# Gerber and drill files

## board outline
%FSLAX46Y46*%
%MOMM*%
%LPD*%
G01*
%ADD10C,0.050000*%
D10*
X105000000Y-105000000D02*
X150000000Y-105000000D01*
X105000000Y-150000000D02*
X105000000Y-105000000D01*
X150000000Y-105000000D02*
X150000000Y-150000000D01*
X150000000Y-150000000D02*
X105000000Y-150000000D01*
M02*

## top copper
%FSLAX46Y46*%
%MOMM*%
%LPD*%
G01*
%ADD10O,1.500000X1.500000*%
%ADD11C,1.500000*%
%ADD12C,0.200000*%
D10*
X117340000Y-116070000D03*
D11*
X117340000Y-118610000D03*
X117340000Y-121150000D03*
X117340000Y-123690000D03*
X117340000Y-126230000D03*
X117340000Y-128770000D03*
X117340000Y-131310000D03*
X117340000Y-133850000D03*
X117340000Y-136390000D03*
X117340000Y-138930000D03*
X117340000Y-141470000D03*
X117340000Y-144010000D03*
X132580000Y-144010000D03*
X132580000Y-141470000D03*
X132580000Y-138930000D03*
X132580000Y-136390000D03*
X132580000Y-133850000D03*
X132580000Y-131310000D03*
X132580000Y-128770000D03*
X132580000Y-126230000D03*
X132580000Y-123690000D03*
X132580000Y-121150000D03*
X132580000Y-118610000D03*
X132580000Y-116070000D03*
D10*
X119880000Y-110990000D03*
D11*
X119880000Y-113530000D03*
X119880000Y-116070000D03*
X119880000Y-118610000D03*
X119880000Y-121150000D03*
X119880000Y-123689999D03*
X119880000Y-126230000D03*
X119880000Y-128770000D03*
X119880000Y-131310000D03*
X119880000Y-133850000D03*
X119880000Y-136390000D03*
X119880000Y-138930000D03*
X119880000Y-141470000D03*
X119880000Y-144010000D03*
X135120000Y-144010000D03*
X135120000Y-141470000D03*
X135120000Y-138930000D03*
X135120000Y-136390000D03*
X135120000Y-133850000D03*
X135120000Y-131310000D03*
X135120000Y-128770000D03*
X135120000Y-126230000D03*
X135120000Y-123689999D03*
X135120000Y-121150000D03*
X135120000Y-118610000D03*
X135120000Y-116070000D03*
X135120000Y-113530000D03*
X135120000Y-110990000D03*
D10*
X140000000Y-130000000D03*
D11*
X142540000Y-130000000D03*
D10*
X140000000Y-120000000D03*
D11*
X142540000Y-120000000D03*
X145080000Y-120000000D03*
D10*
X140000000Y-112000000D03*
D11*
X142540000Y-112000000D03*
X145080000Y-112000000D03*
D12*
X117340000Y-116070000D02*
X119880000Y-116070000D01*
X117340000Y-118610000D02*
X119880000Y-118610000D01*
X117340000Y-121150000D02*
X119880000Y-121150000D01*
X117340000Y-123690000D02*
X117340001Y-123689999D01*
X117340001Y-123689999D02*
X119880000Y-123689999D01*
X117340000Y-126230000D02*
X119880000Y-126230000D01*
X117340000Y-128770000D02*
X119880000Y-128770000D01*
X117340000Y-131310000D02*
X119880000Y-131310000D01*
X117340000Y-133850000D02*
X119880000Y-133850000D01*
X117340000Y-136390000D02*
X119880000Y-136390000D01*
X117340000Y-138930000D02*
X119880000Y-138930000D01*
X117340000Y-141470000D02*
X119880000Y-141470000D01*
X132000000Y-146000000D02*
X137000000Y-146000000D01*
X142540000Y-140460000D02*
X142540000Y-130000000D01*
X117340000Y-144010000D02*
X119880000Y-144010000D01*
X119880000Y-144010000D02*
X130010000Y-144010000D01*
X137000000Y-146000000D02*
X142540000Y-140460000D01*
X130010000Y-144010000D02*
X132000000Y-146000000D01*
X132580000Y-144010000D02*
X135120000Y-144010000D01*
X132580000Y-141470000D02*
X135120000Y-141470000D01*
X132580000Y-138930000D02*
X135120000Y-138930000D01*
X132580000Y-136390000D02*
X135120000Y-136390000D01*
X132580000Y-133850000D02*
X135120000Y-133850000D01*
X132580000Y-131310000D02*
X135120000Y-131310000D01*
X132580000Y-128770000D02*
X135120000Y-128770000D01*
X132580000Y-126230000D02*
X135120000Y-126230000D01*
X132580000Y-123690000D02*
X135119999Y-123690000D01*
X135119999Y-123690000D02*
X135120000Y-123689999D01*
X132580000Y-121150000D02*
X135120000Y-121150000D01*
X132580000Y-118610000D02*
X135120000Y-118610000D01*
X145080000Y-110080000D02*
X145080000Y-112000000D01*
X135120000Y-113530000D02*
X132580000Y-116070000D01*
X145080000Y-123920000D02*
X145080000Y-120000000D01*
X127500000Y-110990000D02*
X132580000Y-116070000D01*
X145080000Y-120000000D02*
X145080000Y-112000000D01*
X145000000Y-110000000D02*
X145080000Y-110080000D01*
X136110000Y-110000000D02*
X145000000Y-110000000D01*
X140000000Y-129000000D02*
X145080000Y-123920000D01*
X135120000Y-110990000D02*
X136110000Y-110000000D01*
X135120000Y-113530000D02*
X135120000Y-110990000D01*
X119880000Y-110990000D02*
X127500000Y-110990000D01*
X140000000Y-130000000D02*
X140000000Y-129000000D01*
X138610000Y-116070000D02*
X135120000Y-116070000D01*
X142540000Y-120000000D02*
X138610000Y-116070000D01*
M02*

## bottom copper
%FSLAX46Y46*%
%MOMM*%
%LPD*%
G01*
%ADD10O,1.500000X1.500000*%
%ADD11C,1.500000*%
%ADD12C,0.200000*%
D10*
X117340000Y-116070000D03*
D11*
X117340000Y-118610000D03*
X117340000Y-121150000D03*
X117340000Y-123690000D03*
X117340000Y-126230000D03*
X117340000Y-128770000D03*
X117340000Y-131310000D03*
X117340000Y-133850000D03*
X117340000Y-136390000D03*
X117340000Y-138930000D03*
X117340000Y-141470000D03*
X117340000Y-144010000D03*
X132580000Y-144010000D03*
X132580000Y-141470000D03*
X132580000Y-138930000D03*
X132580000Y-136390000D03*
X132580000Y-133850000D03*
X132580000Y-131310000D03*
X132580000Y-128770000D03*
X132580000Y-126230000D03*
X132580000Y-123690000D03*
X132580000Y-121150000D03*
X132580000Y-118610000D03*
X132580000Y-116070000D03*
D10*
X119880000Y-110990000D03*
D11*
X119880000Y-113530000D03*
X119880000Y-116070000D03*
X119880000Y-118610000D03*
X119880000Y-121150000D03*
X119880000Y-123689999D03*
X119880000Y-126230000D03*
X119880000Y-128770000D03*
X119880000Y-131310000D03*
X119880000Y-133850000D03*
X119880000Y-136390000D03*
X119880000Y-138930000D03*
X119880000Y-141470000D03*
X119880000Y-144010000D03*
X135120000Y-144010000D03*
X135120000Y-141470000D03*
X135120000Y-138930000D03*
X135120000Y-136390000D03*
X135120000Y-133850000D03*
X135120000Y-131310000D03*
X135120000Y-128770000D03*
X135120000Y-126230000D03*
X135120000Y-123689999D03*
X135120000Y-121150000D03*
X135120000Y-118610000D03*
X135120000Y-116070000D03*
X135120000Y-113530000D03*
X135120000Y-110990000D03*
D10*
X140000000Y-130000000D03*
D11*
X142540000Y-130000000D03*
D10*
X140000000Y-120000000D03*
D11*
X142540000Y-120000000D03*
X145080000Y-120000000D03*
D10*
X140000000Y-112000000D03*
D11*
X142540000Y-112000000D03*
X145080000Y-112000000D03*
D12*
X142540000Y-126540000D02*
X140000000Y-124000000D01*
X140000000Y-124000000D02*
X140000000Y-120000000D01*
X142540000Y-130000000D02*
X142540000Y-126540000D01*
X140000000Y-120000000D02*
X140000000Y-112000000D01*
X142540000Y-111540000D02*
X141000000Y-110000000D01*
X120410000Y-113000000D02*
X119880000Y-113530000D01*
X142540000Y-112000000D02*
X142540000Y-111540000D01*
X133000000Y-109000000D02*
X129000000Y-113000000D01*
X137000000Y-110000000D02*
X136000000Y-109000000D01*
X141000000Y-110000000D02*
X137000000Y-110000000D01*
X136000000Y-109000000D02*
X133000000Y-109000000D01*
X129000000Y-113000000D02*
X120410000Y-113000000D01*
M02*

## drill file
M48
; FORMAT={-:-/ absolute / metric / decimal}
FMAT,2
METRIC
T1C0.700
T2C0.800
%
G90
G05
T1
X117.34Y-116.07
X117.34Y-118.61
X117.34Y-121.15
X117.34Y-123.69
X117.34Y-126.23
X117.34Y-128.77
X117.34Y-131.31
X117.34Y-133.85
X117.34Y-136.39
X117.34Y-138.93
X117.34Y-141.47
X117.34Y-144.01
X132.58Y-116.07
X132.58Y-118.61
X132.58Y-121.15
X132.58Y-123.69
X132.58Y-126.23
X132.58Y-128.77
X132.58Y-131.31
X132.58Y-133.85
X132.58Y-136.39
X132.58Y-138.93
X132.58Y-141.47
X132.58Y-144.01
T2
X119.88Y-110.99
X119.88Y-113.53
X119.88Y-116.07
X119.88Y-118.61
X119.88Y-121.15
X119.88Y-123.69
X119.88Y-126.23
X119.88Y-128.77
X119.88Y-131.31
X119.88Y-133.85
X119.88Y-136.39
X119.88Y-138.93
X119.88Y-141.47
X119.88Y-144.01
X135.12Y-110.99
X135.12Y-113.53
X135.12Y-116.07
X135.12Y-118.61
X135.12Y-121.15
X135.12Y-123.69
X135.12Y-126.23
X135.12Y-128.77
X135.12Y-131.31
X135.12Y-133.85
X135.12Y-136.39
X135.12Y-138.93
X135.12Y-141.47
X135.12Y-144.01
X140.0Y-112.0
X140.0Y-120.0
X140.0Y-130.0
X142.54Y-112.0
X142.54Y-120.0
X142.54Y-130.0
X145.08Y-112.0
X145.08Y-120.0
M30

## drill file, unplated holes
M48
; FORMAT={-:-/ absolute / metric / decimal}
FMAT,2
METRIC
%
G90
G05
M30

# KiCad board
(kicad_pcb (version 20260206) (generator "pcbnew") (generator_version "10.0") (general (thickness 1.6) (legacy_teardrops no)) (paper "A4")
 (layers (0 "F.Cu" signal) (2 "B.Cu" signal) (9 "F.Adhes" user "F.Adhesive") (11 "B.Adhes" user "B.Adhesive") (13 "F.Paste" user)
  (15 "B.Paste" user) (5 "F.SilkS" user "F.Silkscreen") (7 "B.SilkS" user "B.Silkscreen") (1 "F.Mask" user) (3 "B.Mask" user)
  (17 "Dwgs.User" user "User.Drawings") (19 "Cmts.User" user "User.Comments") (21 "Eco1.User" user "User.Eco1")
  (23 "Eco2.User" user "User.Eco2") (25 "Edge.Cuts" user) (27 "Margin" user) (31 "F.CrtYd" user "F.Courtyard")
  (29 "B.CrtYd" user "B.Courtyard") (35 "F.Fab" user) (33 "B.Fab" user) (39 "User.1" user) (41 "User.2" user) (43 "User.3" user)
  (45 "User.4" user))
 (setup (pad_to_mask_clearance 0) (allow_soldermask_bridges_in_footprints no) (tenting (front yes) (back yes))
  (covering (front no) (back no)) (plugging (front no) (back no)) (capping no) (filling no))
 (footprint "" (layer "F.Cu") (at 100 100)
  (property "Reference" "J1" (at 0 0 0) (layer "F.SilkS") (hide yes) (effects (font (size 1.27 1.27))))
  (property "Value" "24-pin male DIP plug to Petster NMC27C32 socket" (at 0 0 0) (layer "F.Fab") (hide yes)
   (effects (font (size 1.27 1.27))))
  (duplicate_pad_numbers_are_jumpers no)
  (pad "1" thru_hole oval (at 17.34 16.07) (size 1.5 1.5) (drill 0.7) (layers "*.Cu" "*.Mask") (remove_unused_layers no) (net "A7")
   (thermal_bridge_angle 45))
  (pad "2" thru_hole circle (at 17.34 18.61) (size 1.5 1.5) (drill 0.7) (layers "*.Cu" "*.Mask") (remove_unused_layers no) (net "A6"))
  (pad "3" thru_hole circle (at 17.34 21.15) (size 1.5 1.5) (drill 0.7) (layers "*.Cu" "*.Mask") (remove_unused_layers no) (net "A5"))
  (pad "4" thru_hole circle (at 17.34 23.69) (size 1.5 1.5) (drill 0.7) (layers "*.Cu" "*.Mask") (remove_unused_layers no) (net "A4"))
  (pad "5" thru_hole circle (at 17.34 26.23) (size 1.5 1.5) (drill 0.7) (layers "*.Cu" "*.Mask") (remove_unused_layers no) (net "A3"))
  (pad "6" thru_hole circle (at 17.34 28.77) (size 1.5 1.5) (drill 0.7) (layers "*.Cu" "*.Mask") (remove_unused_layers no) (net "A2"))
  (pad "7" thru_hole circle (at 17.34 31.31) (size 1.5 1.5) (drill 0.7) (layers "*.Cu" "*.Mask") (remove_unused_layers no) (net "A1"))
  (pad "8" thru_hole circle (at 17.34 33.85) (size 1.5 1.5) (drill 0.7) (layers "*.Cu" "*.Mask") (remove_unused_layers no) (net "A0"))
  (pad "9" thru_hole circle (at 17.34 36.39) (size 1.5 1.5) (drill 0.7) (layers "*.Cu" "*.Mask") (remove_unused_layers no) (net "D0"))
  (pad "10" thru_hole circle (at 17.34 38.93) (size 1.5 1.5) (drill 0.7) (layers "*.Cu" "*.Mask") (remove_unused_layers no) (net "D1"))
  (pad "11" thru_hole circle (at 17.34 41.47) (size 1.5 1.5) (drill 0.7) (layers "*.Cu" "*.Mask") (remove_unused_layers no) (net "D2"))
  (pad "12" thru_hole circle (at 17.34 44.01) (size 1.5 1.5) (drill 0.7) (layers "*.Cu" "*.Mask") (remove_unused_layers no) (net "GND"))
  (pad "13" thru_hole circle (at 32.58 44.01) (size 1.5 1.5) (drill 0.7) (layers "*.Cu" "*.Mask") (remove_unused_layers no) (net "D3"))
  (pad "14" thru_hole circle (at 32.58 41.47) (size 1.5 1.5) (drill 0.7) (layers "*.Cu" "*.Mask") (remove_unused_layers no) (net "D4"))
  (pad "15" thru_hole circle (at 32.58 38.93) (size 1.5 1.5) (drill 0.7) (layers "*.Cu" "*.Mask") (remove_unused_layers no) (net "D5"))
  (pad "16" thru_hole circle (at 32.58 36.39) (size 1.5 1.5) (drill 0.7) (layers "*.Cu" "*.Mask") (remove_unused_layers no) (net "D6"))
  (pad "17" thru_hole circle (at 32.58 33.85) (size 1.5 1.5) (drill 0.7) (layers "*.Cu" "*.Mask") (remove_unused_layers no) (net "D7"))
  (pad "18" thru_hole circle (at 32.58 31.31) (size 1.5 1.5) (drill 0.7) (layers "*.Cu" "*.Mask") (remove_unused_layers no) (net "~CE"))
  (pad "19" thru_hole circle (at 32.58 28.77) (size 1.5 1.5) (drill 0.7) (layers "*.Cu" "*.Mask") (remove_unused_layers no) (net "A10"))
  (pad "20" thru_hole circle (at 32.58 26.23) (size 1.5 1.5) (drill 0.7) (layers "*.Cu" "*.Mask") (remove_unused_layers no) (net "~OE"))
  (pad "21" thru_hole circle (at 32.58 23.69) (size 1.5 1.5) (drill 0.7) (layers "*.Cu" "*.Mask") (remove_unused_layers no) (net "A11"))
  (pad "22" thru_hole circle (at 32.58 21.15) (size 1.5 1.5) (drill 0.7) (layers "*.Cu" "*.Mask") (remove_unused_layers no) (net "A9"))
  (pad "23" thru_hole circle (at 32.58 18.61) (size 1.5 1.5) (drill 0.7) (layers "*.Cu" "*.Mask") (remove_unused_layers no) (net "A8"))
  (pad "24" thru_hole circle (at 32.58 16.07) (size 1.5 1.5) (drill 0.7) (layers "*.Cu" "*.Mask") (remove_unused_layers no) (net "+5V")))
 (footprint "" (layer "F.Cu") (at 100 100)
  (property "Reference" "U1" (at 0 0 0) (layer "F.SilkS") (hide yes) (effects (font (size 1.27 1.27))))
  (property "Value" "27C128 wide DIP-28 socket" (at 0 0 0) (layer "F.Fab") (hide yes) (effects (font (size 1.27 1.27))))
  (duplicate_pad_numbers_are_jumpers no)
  (pad "1" thru_hole oval (at 19.88 10.99) (size 1.5 1.5) (drill 0.8) (layers "*.Cu" "*.Mask") (remove_unused_layers no) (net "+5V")
   (thermal_bridge_angle 45))
  (pad "2" thru_hole circle (at 19.88 13.53) (size 1.5 1.5) (drill 0.8) (layers "*.Cu" "*.Mask") (remove_unused_layers no) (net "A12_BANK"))
  (pad "3" thru_hole circle (at 19.88 16.07) (size 1.5 1.5) (drill 0.8) (layers "*.Cu" "*.Mask") (remove_unused_layers no) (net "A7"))
  (pad "4" thru_hole circle (at 19.88 18.61) (size 1.5 1.5) (drill 0.8) (layers "*.Cu" "*.Mask") (remove_unused_layers no) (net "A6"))
  (pad "5" thru_hole circle (at 19.88 21.15) (size 1.5 1.5) (drill 0.8) (layers "*.Cu" "*.Mask") (remove_unused_layers no) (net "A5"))
  (pad "6" thru_hole circle (at 19.88 23.689999) (size 1.5 1.5) (drill 0.8) (layers "*.Cu" "*.Mask") (remove_unused_layers no) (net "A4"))
  (pad "7" thru_hole circle (at 19.88 26.23) (size 1.5 1.5) (drill 0.8) (layers "*.Cu" "*.Mask") (remove_unused_layers no) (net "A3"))
  (pad "8" thru_hole circle (at 19.88 28.77) (size 1.5 1.5) (drill 0.8) (layers "*.Cu" "*.Mask") (remove_unused_layers no) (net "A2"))
  (pad "9" thru_hole circle (at 19.88 31.31) (size 1.5 1.5) (drill 0.8) (layers "*.Cu" "*.Mask") (remove_unused_layers no) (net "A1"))
  (pad "10" thru_hole circle (at 19.88 33.85) (size 1.5 1.5) (drill 0.8) (layers "*.Cu" "*.Mask") (remove_unused_layers no) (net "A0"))
  (pad "11" thru_hole circle (at 19.88 36.39) (size 1.5 1.5) (drill 0.8) (layers "*.Cu" "*.Mask") (remove_unused_layers no) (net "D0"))
  (pad "12" thru_hole circle (at 19.88 38.93) (size 1.5 1.5) (drill 0.8) (layers "*.Cu" "*.Mask") (remove_unused_layers no) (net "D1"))
  (pad "13" thru_hole circle (at 19.88 41.47) (size 1.5 1.5) (drill 0.8) (layers "*.Cu" "*.Mask") (remove_unused_layers no) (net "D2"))
  (pad "14" thru_hole circle (at 19.88 44.01) (size 1.5 1.5) (drill 0.8) (layers "*.Cu" "*.Mask") (remove_unused_layers no) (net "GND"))
  (pad "15" thru_hole circle (at 35.12 44.01) (size 1.5 1.5) (drill 0.8) (layers "*.Cu" "*.Mask") (remove_unused_layers no) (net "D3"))
  (pad "16" thru_hole circle (at 35.12 41.47) (size 1.5 1.5) (drill 0.8) (layers "*.Cu" "*.Mask") (remove_unused_layers no) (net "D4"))
  (pad "17" thru_hole circle (at 35.12 38.93) (size 1.5 1.5) (drill 0.8) (layers "*.Cu" "*.Mask") (remove_unused_layers no) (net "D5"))
  (pad "18" thru_hole circle (at 35.12 36.39) (size 1.5 1.5) (drill 0.8) (layers "*.Cu" "*.Mask") (remove_unused_layers no) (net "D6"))
  (pad "19" thru_hole circle (at 35.12 33.85) (size 1.5 1.5) (drill 0.8) (layers "*.Cu" "*.Mask") (remove_unused_layers no) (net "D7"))
  (pad "20" thru_hole circle (at 35.12 31.31) (size 1.5 1.5) (drill 0.8) (layers "*.Cu" "*.Mask") (remove_unused_layers no) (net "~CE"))
  (pad "21" thru_hole circle (at 35.12 28.77) (size 1.5 1.5) (drill 0.8) (layers "*.Cu" "*.Mask") (remove_unused_layers no) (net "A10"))
  (pad "22" thru_hole circle (at 35.12 26.23) (size 1.5 1.5) (drill 0.8) (layers "*.Cu" "*.Mask") (remove_unused_layers no) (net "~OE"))
  (pad "23" thru_hole circle (at 35.12 23.689999) (size 1.5 1.5) (drill 0.8) (layers "*.Cu" "*.Mask") (remove_unused_layers no) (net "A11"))
  (pad "24" thru_hole circle (at 35.12 21.15) (size 1.5 1.5) (drill 0.8) (layers "*.Cu" "*.Mask") (remove_unused_layers no) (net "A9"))
  (pad "25" thru_hole circle (at 35.12 18.61) (size 1.5 1.5) (drill 0.8) (layers "*.Cu" "*.Mask") (remove_unused_layers no) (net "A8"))
  (pad "26" thru_hole circle (at 35.12 16.07) (size 1.5 1.5) (drill 0.8) (layers "*.Cu" "*.Mask") (remove_unused_layers no) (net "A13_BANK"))
  (pad "27" thru_hole circle (at 35.12 13.53) (size 1.5 1.5) (drill 0.8) (layers "*.Cu" "*.Mask") (remove_unused_layers no) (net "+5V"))
  (pad "28" thru_hole circle (at 35.12 10.99) (size 1.5 1.5) (drill 0.8) (layers "*.Cu" "*.Mask") (remove_unused_layers no) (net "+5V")))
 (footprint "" (layer "F.Cu") (at 100 100)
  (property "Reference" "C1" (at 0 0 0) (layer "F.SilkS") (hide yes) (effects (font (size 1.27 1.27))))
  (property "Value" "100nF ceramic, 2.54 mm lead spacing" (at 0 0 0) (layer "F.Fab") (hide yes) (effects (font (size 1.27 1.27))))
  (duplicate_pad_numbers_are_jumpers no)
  (pad "1" thru_hole oval (at 40 30) (size 1.5 1.5) (drill 0.8) (layers "*.Cu" "*.Mask") (remove_unused_layers no) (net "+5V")
   (thermal_bridge_angle 45))
  (pad "2" thru_hole circle (at 42.54 30) (size 1.5 1.5) (drill 0.8) (layers "*.Cu" "*.Mask") (remove_unused_layers no) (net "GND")))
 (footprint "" (layer "F.Cu") (at 100 100)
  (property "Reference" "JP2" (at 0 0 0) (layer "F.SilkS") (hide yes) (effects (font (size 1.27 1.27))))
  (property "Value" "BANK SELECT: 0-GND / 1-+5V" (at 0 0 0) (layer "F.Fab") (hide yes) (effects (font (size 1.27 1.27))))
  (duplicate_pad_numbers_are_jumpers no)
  (pad "1" thru_hole oval (at 40 20) (size 1.5 1.5) (drill 0.8) (layers "*.Cu" "*.Mask") (remove_unused_layers no) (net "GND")
   (thermal_bridge_angle 45))
  (pad "2" thru_hole circle (at 42.54 20) (size 1.5 1.5) (drill 0.8) (layers "*.Cu" "*.Mask") (remove_unused_layers no) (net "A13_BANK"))
  (pad "3" thru_hole circle (at 45.08 20) (size 1.5 1.5) (drill 0.8) (layers "*.Cu" "*.Mask") (remove_unused_layers no) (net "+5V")))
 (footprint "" (layer "F.Cu") (at 100 100)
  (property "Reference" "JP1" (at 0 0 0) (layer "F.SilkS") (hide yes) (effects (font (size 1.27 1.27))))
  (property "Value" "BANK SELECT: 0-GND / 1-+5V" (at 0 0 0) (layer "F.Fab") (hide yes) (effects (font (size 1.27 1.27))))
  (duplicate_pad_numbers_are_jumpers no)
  (pad "1" thru_hole oval (at 40 12) (size 1.5 1.5) (drill 0.8) (layers "*.Cu" "*.Mask") (remove_unused_layers no) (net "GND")
   (thermal_bridge_angle 45))
  (pad "2" thru_hole circle (at 42.54 12) (size 1.5 1.5) (drill 0.8) (layers "*.Cu" "*.Mask") (remove_unused_layers no) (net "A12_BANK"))
  (pad "3" thru_hole circle (at 45.08 12) (size 1.5 1.5) (drill 0.8) (layers "*.Cu" "*.Mask") (remove_unused_layers no) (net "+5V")))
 (gr_line (start 105 105) (end 150 105) (stroke (width 0.05) (type default)) (layer "Edge.Cuts"))
 (gr_line (start 105 150) (end 105 105) (stroke (width 0.05) (type default)) (layer "Edge.Cuts"))
 (gr_line (start 150 105) (end 150 150) (stroke (width 0.05) (type default)) (layer "Edge.Cuts"))
 (gr_line (start 150 150) (end 105 150) (stroke (width 0.05) (type default)) (layer "Edge.Cuts"))
 (segment (start 117.34 116.07) (end 119.88 116.07) (width 0.2) (layer "F.Cu") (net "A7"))
 (segment (start 117.34 118.61) (end 119.88 118.61) (width 0.2) (layer "F.Cu") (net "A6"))
 (segment (start 117.34 121.15) (end 119.88 121.15) (width 0.2) (layer "F.Cu") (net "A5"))
 (segment (start 117.34 123.69) (end 117.340001 123.689999) (width 0.2) (layer "F.Cu") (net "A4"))
 (segment (start 117.340001 123.689999) (end 119.88 123.689999) (width 0.2) (layer "F.Cu") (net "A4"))
 (segment (start 117.34 126.23) (end 119.88 126.23) (width 0.2) (layer "F.Cu") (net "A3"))
 (segment (start 117.34 128.77) (end 119.88 128.77) (width 0.2) (layer "F.Cu") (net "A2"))
 (segment (start 117.34 131.31) (end 119.88 131.31) (width 0.2) (layer "F.Cu") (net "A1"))
 (segment (start 117.34 133.85) (end 119.88 133.85) (width 0.2) (layer "F.Cu") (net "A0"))
 (segment (start 117.34 136.39) (end 119.88 136.39) (width 0.2) (layer "F.Cu") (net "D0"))
 (segment (start 117.34 138.93) (end 119.88 138.93) (width 0.2) (layer "F.Cu") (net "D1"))
 (segment (start 117.34 141.47) (end 119.88 141.47) (width 0.2) (layer "F.Cu") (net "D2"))
 (segment (start 132 146) (end 137 146) (width 0.2) (layer "F.Cu") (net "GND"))
 (segment (start 142.54 140.46) (end 142.54 130) (width 0.2) (layer "F.Cu") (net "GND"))
 (segment (start 117.34 144.01) (end 119.88 144.01) (width 0.2) (layer "F.Cu") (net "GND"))
 (segment (start 119.88 144.01) (end 130.01 144.01) (width 0.2) (layer "F.Cu") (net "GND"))
 (segment (start 137 146) (end 142.54 140.46) (width 0.2) (layer "F.Cu") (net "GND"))
 (segment (start 130.01 144.01) (end 132 146) (width 0.2) (layer "F.Cu") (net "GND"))
 (segment (start 142.54 126.54) (end 140 124) (width 0.2) (layer "B.Cu") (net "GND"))
 (segment (start 140 124) (end 140 120) (width 0.2) (layer "B.Cu") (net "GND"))
 (segment (start 142.54 130) (end 142.54 126.54) (width 0.2) (layer "B.Cu") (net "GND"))
 (segment (start 140 120) (end 140 112) (width 0.2) (layer "B.Cu") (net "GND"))
 (segment (start 132.58 144.01) (end 135.12 144.01) (width 0.2) (layer "F.Cu") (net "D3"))
 (segment (start 132.58 141.47) (end 135.12 141.47) (width 0.2) (layer "F.Cu") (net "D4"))
 (segment (start 132.58 138.93) (end 135.12 138.93) (width 0.2) (layer "F.Cu") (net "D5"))
 (segment (start 132.58 136.39) (end 135.12 136.39) (width 0.2) (layer "F.Cu") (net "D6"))
 (segment (start 132.58 133.85) (end 135.12 133.85) (width 0.2) (layer "F.Cu") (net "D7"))
 (segment (start 132.58 131.31) (end 135.12 131.31) (width 0.2) (layer "F.Cu") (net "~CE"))
 (segment (start 132.58 128.77) (end 135.12 128.77) (width 0.2) (layer "F.Cu") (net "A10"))
 (segment (start 132.58 126.23) (end 135.12 126.23) (width 0.2) (layer "F.Cu") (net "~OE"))
 (segment (start 132.58 123.69) (end 135.119999 123.69) (width 0.2) (layer "F.Cu") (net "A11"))
 (segment (start 135.119999 123.69) (end 135.12 123.689999) (width 0.2) (layer "F.Cu") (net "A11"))
 (segment (start 132.58 121.15) (end 135.12 121.15) (width 0.2) (layer "F.Cu") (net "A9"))
 (segment (start 132.58 118.61) (end 135.12 118.61) (width 0.2) (layer "F.Cu") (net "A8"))
 (segment (start 145.08 110.08) (end 145.08 112) (width 0.2) (layer "F.Cu") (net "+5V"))
 (segment (start 135.12 113.53) (end 132.58 116.07) (width 0.2) (layer "F.Cu") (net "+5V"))
 (segment (start 145.08 123.92) (end 145.08 120) (width 0.2) (layer "F.Cu") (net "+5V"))
 (segment (start 127.5 110.99) (end 132.58 116.07) (width 0.2) (layer "F.Cu") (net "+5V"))
 (segment (start 145.08 120) (end 145.08 112) (width 0.2) (layer "F.Cu") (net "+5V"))
 (segment (start 145 110) (end 145.08 110.08) (width 0.2) (layer "F.Cu") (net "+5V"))
 (segment (start 136.11 110) (end 145 110) (width 0.2) (layer "F.Cu") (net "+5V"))
 (segment (start 140 129) (end 145.08 123.92) (width 0.2) (layer "F.Cu") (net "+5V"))
 (segment (start 135.12 110.99) (end 136.11 110) (width 0.2) (layer "F.Cu") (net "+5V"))
 (segment (start 135.12 113.53) (end 135.12 110.99) (width 0.2) (layer "F.Cu") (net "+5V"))
 (segment (start 119.88 110.99) (end 127.5 110.99) (width 0.2) (layer "F.Cu") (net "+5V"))
 (segment (start 140 130) (end 140 129) (width 0.2) (layer "F.Cu") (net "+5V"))
 (segment (start 142.54 111.54) (end 141 110) (width 0.2) (layer "B.Cu") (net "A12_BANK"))
 (segment (start 120.41 113) (end 119.88 113.53) (width 0.2) (layer "B.Cu") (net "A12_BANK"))
 (segment (start 142.54 112) (end 142.54 111.54) (width 0.2) (layer "B.Cu") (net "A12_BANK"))
 (segment (start 133 109) (end 129 113) (width 0.2) (layer "B.Cu") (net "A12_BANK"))
 (segment (start 137 110) (end 136 109) (width 0.2) (layer "B.Cu") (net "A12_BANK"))
 (segment (start 141 110) (end 137 110) (width 0.2) (layer "B.Cu") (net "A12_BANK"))
 (segment (start 136 109) (end 133 109) (width 0.2) (layer "B.Cu") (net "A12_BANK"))
 (segment (start 129 113) (end 120.41 113) (width 0.2) (layer "B.Cu") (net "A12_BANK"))
 (segment (start 138.61 116.07) (end 135.12 116.07) (width 0.2) (layer "F.Cu") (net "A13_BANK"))
 (segment (start 142.54 120) (end 138.61 116.07) (width 0.2) (layer "F.Cu") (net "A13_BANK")))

